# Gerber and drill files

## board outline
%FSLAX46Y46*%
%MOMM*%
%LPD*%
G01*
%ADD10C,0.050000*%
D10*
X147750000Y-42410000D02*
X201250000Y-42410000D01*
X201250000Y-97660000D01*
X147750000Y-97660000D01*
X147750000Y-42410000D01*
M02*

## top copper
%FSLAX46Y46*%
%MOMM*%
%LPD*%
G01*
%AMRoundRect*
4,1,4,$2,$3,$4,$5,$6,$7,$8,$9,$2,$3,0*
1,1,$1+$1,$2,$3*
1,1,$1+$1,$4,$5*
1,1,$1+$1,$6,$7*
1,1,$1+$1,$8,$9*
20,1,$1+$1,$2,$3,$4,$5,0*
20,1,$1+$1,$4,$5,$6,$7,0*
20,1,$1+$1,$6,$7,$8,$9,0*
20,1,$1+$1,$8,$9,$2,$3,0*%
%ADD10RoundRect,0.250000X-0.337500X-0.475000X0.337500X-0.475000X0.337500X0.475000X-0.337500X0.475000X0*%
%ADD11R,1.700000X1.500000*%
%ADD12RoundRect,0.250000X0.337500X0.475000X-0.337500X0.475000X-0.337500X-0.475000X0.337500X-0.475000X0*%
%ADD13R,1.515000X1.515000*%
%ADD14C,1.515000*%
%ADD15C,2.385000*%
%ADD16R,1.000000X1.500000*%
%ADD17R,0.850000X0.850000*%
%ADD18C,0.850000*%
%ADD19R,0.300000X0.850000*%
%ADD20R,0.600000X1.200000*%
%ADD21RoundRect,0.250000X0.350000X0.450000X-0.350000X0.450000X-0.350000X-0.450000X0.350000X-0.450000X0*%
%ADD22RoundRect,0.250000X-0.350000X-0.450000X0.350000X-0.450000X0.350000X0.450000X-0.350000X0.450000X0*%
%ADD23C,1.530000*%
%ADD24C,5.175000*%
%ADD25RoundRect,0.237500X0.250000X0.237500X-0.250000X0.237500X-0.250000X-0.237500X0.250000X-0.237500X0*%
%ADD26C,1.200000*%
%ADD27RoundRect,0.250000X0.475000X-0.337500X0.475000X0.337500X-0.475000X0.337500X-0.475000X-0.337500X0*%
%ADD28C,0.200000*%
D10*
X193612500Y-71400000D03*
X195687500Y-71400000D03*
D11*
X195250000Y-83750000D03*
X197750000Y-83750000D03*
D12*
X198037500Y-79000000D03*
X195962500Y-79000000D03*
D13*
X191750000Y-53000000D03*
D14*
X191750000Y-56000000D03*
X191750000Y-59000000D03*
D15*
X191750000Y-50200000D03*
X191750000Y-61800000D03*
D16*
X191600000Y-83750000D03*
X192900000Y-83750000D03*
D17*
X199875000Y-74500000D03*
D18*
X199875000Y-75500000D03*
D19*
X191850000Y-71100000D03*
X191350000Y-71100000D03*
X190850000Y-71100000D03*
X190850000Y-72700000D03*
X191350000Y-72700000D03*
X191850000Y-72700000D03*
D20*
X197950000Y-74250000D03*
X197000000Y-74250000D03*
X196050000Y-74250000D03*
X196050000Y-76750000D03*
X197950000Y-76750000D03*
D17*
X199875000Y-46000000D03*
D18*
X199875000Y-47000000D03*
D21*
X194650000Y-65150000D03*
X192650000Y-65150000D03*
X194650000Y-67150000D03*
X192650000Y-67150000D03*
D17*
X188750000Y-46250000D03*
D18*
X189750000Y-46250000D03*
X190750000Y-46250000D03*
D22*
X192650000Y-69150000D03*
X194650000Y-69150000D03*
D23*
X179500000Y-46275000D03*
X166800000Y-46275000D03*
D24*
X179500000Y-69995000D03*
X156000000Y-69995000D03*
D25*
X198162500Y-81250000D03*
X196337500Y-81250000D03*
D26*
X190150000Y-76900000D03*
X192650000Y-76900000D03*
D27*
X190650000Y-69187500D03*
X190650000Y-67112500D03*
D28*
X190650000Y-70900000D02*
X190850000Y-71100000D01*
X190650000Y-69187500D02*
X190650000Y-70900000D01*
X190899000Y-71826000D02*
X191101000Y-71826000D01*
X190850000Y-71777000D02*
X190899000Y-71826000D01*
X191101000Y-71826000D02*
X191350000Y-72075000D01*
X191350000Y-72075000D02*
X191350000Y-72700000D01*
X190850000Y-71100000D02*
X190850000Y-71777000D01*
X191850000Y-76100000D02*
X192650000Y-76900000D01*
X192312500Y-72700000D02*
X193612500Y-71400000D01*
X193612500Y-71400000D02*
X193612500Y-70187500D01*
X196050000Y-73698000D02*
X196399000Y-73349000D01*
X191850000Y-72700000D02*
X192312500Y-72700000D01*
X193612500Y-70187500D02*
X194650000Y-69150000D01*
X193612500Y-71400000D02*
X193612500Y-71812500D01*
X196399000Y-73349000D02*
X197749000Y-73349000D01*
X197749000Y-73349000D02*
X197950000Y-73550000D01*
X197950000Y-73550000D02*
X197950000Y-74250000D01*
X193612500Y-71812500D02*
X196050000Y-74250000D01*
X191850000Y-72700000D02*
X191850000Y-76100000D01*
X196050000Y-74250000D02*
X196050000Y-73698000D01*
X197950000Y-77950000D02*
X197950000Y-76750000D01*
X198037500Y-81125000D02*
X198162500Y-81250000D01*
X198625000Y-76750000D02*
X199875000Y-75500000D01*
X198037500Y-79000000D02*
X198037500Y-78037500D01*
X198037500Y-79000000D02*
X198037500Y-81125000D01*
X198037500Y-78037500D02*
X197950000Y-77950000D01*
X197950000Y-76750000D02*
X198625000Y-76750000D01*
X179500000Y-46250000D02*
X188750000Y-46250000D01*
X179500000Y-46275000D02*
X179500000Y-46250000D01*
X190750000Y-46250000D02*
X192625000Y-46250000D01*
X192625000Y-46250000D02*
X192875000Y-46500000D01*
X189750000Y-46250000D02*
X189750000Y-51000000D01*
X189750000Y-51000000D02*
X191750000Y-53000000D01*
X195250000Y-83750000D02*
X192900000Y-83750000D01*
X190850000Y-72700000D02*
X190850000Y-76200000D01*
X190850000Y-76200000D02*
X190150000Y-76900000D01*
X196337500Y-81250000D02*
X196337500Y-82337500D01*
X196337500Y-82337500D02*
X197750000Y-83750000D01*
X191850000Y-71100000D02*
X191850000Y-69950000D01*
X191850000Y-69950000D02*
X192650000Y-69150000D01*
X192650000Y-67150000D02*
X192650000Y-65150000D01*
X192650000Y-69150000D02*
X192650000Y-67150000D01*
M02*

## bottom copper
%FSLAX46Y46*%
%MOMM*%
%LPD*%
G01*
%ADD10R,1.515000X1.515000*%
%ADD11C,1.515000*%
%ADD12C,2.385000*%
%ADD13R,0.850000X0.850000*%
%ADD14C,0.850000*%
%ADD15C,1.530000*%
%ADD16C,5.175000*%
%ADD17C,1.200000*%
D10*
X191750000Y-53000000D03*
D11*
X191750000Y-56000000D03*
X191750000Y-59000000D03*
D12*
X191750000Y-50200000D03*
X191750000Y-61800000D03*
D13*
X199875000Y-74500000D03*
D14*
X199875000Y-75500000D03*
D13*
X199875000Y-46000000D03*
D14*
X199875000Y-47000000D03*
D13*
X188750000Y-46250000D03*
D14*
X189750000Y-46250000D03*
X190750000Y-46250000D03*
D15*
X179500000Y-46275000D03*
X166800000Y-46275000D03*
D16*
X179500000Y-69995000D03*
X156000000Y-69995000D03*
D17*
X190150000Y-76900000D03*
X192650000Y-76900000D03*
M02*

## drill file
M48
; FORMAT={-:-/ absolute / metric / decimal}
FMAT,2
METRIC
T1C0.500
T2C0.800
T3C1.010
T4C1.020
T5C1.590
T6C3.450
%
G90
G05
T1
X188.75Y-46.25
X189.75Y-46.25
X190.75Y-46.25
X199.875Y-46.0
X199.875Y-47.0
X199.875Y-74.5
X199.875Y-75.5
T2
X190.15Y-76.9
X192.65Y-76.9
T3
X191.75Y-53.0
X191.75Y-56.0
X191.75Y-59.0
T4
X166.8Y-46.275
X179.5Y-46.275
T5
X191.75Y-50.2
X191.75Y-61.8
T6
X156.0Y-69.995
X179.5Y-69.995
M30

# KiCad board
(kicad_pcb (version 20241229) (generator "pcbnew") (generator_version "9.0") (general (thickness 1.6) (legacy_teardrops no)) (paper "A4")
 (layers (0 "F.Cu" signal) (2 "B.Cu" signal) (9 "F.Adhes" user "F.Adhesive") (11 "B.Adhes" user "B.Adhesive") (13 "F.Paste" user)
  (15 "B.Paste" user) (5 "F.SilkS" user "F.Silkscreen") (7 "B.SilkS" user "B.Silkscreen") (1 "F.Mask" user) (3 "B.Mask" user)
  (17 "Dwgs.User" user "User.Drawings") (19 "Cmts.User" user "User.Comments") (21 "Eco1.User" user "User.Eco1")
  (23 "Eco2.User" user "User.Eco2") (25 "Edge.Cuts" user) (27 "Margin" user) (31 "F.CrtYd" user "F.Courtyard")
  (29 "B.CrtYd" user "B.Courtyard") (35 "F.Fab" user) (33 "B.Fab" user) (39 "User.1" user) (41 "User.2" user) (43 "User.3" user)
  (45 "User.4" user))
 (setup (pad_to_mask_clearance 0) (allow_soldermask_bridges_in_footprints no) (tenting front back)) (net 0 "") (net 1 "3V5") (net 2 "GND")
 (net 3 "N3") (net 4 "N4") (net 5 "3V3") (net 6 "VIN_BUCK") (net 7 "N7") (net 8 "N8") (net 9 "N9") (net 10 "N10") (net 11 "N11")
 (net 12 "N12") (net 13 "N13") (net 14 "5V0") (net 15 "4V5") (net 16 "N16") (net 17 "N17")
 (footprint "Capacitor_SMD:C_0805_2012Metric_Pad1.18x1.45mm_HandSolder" (layer "F.Cu") (at 194.65 71.4)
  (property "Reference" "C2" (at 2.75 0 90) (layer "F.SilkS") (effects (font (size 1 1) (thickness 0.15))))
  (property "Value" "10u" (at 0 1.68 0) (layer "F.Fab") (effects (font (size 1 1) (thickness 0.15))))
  (pad "1" smd roundrect (at -1.0375 0) (size 1.175 1.45) (layers "F.Cu" "F.Mask" "F.Paste") (roundrect_rratio 0.212766) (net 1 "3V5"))
  (pad "2" smd roundrect (at 1.0375 0) (size 1.175 1.45) (layers "F.Cu" "F.Mask" "F.Paste") (roundrect_rratio 0.212766) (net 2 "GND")))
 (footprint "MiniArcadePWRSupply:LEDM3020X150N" (layer "F.Cu") (at 196.5 83.75)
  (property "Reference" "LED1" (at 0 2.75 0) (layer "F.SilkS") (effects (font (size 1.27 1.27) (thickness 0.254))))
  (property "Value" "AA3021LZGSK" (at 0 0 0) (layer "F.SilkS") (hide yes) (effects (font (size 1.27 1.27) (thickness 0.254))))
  (pad "1" smd rect (at -1.25 0 90) (size 1.5 1.7) (layers "F.Cu" "F.Mask" "F.Paste") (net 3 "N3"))
  (pad "2" smd rect (at 1.25 0 90) (size 1.5 1.7) (layers "F.Cu" "F.Mask" "F.Paste") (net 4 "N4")))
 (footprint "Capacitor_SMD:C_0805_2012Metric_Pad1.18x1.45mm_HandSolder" (layer "F.Cu") (at 197 79 180)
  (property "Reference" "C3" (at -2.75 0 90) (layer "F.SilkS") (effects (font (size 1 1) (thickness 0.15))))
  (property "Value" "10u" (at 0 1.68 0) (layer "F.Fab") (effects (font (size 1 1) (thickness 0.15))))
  (pad "1" smd roundrect (at -1.0375 0 180) (size 1.175 1.45) (layers "F.Cu" "F.Mask" "F.Paste") (roundrect_rratio 0.212766) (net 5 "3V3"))
  (pad "2" smd roundrect (at 1.0375 0 180) (size 1.175 1.45) (layers "F.Cu" "F.Mask" "F.Paste") (roundrect_rratio 0.212766) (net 2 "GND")))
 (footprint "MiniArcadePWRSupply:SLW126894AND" (layer "F.Cu") (at 191.75 53 -90)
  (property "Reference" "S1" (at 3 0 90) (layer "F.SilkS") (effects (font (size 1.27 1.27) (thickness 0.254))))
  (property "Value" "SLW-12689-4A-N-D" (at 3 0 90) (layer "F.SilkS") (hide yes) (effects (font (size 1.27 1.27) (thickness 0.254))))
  (pad "1" thru_hole rect (at 0 0 270) (size 1.515 1.515) (drill 1.01) (layers "*.Cu" "*.Mask") (remove_unused_layers no) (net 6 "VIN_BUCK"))
  (pad "2" thru_hole circle (at 3 0 270) (size 1.515 1.515) (drill 1.01) (layers "*.Cu" "*.Mask") (remove_unused_layers no) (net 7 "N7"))
  (pad "3" thru_hole circle (at 6 0 270) (size 1.515 1.515) (drill 1.01) (layers "*.Cu" "*.Mask") (remove_unused_layers no) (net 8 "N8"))
  (pad "4" thru_hole circle (at -2.8 0 270) (size 2.385 2.385) (drill 1.59) (layers "*.Cu" "*.Mask") (remove_unused_layers no) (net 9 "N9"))
  (pad "5" thru_hole circle (at 8.8 0 270) (size 2.385 2.385) (drill 1.59) (layers "*.Cu" "*.Mask") (remove_unused_layers no) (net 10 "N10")))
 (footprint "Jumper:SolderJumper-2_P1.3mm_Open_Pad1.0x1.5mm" (layer "F.Cu") (at 192.25 83.75)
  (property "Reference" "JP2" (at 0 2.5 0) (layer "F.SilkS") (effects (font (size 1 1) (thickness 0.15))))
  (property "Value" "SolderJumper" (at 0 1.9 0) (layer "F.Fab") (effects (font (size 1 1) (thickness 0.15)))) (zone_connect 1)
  (pad "1" smd rect (at -0.65 0) (size 1 1.5) (layers "F.Cu" "F.Mask") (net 2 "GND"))
  (pad "2" smd rect (at 0.65 0) (size 1 1.5) (layers "F.Cu" "F.Mask") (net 3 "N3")))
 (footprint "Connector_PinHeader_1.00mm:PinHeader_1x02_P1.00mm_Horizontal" (layer "F.Cu") (at 199.875 74.5)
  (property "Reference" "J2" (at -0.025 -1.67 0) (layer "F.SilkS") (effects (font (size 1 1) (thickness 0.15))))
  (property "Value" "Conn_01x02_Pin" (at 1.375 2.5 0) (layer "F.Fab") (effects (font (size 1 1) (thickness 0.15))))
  (pad "1" thru_hole rect (at 0 0) (size 0.85 0.85) (drill 0.5) (layers "*.Cu" "*.Mask") (remove_unused_layers no) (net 2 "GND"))
  (pad "2" thru_hole circle (at 0 1) (size 0.85 0.85) (drill 0.5) (layers "*.Cu" "*.Mask") (remove_unused_layers no) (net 5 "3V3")))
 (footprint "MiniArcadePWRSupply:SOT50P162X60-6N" (layer "F.Cu") (at 191.35 71.9 -90)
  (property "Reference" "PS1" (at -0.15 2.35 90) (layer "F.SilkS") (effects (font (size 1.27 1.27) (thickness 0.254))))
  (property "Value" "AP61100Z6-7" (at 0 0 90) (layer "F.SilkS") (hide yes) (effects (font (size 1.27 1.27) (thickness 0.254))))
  (pad "1" smd rect (at -0.8 -0.5) (size 0.3 0.85) (layers "F.Cu" "F.Mask" "F.Paste") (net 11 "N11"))
  (pad "2" smd rect (at -0.8 0) (size 0.3 0.85) (layers "F.Cu" "F.Mask" "F.Paste") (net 2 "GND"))
  (pad "3" smd rect (at -0.8 0.5) (size 0.3 0.85) (layers "F.Cu" "F.Mask" "F.Paste") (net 7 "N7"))
  (pad "4" smd rect (at 0.8 0.5) (size 0.3 0.85) (layers "F.Cu" "F.Mask" "F.Paste") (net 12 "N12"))
  (pad "5" smd rect (at 0.8 0) (size 0.3 0.85) (layers "F.Cu" "F.Mask" "F.Paste") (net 7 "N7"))
  (pad "6" smd rect (at 0.8 -0.5) (size 0.3 0.85) (layers "F.Cu" "F.Mask" "F.Paste") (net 1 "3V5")))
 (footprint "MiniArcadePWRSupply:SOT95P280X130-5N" (layer "F.Cu") (at 197 75.5 -90)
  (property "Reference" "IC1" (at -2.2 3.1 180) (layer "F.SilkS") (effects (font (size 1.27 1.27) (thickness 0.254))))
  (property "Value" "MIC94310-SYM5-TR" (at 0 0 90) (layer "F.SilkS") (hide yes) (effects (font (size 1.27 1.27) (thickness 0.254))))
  (pad "1" smd rect (at -1.25 -0.95) (size 0.6 1.2) (layers "F.Cu" "F.Mask" "F.Paste") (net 1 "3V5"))
  (pad "2" smd rect (at -1.25 0) (size 0.6 1.2) (layers "F.Cu" "F.Mask" "F.Paste") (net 2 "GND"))
  (pad "3" smd rect (at -1.25 0.95) (size 0.6 1.2) (layers "F.Cu" "F.Mask" "F.Paste") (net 1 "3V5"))
  (pad "4" smd rect (at 1.25 0.95) (size 0.6 1.2) (layers "F.Cu" "F.Mask" "F.Paste") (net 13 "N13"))
  (pad "5" smd rect (at 1.25 -0.95) (size 0.6 1.2) (layers "F.Cu" "F.Mask" "F.Paste") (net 5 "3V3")))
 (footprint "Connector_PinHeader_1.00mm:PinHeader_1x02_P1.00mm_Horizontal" (layer "F.Cu") (at 199.875 46)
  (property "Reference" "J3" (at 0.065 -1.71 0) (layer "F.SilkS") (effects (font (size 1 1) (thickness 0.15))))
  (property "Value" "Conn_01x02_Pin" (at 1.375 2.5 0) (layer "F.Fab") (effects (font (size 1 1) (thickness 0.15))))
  (pad "1" thru_hole rect (at 0 0) (size 0.85 0.85) (drill 0.5) (layers "*.Cu" "*.Mask") (remove_unused_layers no) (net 2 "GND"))
  (pad "2" thru_hole circle (at 0 1) (size 0.85 0.85) (drill 0.5) (layers "*.Cu" "*.Mask") (remove_unused_layers no) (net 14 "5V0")))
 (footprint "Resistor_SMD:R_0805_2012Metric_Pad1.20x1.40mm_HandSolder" (layer "F.Cu") (at 193.65 65.15 180)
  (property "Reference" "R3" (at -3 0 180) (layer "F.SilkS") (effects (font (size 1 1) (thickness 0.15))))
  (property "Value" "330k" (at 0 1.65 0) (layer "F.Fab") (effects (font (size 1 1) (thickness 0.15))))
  (pad "1" smd roundrect (at -1 0 180) (size 1.2 1.4) (layers "F.Cu" "F.Mask" "F.Paste") (roundrect_rratio 0.208333) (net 2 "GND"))
  (pad "2" smd roundrect (at 1 0 180) (size 1.2 1.4) (layers "F.Cu" "F.Mask" "F.Paste") (roundrect_rratio 0.208333) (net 11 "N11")))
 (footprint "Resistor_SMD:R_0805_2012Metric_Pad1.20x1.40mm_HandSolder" (layer "F.Cu") (at 193.65 67.15 180)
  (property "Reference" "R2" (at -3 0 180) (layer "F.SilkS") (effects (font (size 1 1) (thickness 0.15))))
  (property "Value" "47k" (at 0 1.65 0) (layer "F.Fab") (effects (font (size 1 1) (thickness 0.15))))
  (pad "1" smd roundrect (at -1 0 180) (size 1.2 1.4) (layers "F.Cu" "F.Mask" "F.Paste") (roundrect_rratio 0.208333) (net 2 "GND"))
  (pad "2" smd roundrect (at 1 0 180) (size 1.2 1.4) (layers "F.Cu" "F.Mask" "F.Paste") (roundrect_rratio 0.208333) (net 11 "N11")))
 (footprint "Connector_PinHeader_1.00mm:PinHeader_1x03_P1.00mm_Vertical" (layer "F.Cu") (at 188.75 46.25 90)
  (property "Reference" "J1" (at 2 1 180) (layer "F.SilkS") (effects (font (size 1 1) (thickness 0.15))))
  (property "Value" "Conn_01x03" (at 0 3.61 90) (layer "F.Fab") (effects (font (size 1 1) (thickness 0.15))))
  (pad "1" thru_hole rect (at 0 0 90) (size 0.85 0.85) (drill 0.5) (layers "*.Cu" "*.Mask") (remove_unused_layers no) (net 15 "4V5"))
  (pad "2" thru_hole circle (at 0 1 90) (size 0.85 0.85) (drill 0.5) (layers "*.Cu" "*.Mask") (remove_unused_layers no) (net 6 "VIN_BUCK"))
  (pad "3" thru_hole circle (at 0 2 90) (size 0.85 0.85) (drill 0.5) (layers "*.Cu" "*.Mask") (remove_unused_layers no) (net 14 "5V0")))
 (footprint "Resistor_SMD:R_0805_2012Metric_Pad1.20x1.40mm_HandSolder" (layer "F.Cu") (at 193.65 69.15)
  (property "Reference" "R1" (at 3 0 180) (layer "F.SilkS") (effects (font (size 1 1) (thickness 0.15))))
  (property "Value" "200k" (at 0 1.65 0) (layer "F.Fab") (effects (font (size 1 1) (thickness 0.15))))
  (pad "1" smd roundrect (at -1 0) (size 1.2 1.4) (layers "F.Cu" "F.Mask" "F.Paste") (roundrect_rratio 0.208333) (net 11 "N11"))
  (pad "2" smd roundrect (at 1 0) (size 1.2 1.4) (layers "F.Cu" "F.Mask" "F.Paste") (roundrect_rratio 0.208333) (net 1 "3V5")))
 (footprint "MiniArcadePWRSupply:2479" (layer "F.Cu") (at 167.75 70 90)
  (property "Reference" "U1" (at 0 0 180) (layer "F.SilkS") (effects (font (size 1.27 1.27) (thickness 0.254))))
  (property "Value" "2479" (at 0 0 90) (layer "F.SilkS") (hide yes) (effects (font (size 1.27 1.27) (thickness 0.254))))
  (pad "1" thru_hole circle (at 23.725 11.75 90) (size 1.53 1.53) (drill 1.02) (layers "*.Cu" "*.Mask") (remove_unused_layers no)
   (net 15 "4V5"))
  (pad "2" thru_hole circle (at 23.725 -0.95 90) (size 1.53 1.53) (drill 1.02) (layers "*.Cu" "*.Mask") (remove_unused_layers no)
   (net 2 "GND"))
  (pad "3" thru_hole circle (at 0.005 11.75 90) (size 5.175 5.175) (drill 3.45) (layers "*.Cu" "*.Mask") (remove_unused_layers no)
   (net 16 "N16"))
  (pad "4" thru_hole circle (at 0.005 -11.75 90) (size 5.175 5.175) (drill 3.45) (layers "*.Cu" "*.Mask") (remove_unused_layers no)
   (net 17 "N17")))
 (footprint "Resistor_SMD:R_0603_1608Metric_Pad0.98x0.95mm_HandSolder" (layer "F.Cu") (at 197.25 81.25 180)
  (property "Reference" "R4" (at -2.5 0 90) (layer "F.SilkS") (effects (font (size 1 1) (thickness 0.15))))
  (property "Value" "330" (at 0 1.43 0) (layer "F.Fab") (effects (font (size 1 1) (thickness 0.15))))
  (pad "1" smd roundrect (at -0.9125 0 180) (size 0.975 0.95) (layers "F.Cu" "F.Mask" "F.Paste") (roundrect_rratio 0.25) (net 5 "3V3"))
  (pad "2" smd roundrect (at 0.9125 0 180) (size 0.975 0.95) (layers "F.Cu" "F.Mask" "F.Paste") (roundrect_rratio 0.25) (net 4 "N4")))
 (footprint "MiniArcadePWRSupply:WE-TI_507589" (layer "F.Cu") (at 191.4 76.9)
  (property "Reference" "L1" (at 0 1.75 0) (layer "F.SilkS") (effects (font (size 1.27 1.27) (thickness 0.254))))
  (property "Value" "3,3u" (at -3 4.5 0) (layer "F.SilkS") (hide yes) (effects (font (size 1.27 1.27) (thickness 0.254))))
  (pad "1" thru_hole circle (at -1.25 0) (size 1.2 1.2) (drill 0.8) (layers "*.Cu" "*.Mask") (remove_unused_layers no) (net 12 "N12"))
  (pad "2" thru_hole circle (at 1.25 0) (size 1.2 1.2) (drill 0.8) (layers "*.Cu" "*.Mask") (remove_unused_layers no) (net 1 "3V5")))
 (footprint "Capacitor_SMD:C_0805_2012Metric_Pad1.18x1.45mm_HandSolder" (layer "F.Cu") (at 190.65 68.15 90)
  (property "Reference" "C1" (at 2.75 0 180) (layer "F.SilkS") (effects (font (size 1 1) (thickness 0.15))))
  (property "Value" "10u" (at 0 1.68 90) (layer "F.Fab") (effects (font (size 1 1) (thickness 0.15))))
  (pad "1" smd roundrect (at -1.0375 0 90) (size 1.175 1.45) (layers "F.Cu" "F.Mask" "F.Paste") (roundrect_rratio 0.212766) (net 7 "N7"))
  (pad "2" smd roundrect (at 1.0375 0 90) (size 1.175 1.45) (layers "F.Cu" "F.Mask" "F.Paste") (roundrect_rratio 0.212766) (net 2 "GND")))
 (gr_rect (start 147.75 42.41) (end 201.25 97.66) (stroke (width 0.05) (type default)) (fill no) (layer "Edge.Cuts"))
 (segment (start 190.65 70.9) (end 190.85 71.1) (width 0.2) (layer "F.Cu") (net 7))
 (segment (start 190.65 69.1875) (end 190.65 70.9) (width 0.2) (layer "F.Cu") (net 7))
 (segment (start 190.899 71.826) (end 191.101 71.826) (width 0.2) (layer "F.Cu") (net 7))
 (segment (start 190.85 71.777) (end 190.899 71.826) (width 0.2) (layer "F.Cu") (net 7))
 (segment (start 191.101 71.826) (end 191.35 72.075) (width 0.2) (layer "F.Cu") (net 7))
 (segment (start 191.35 72.075) (end 191.35 72.7) (width 0.2) (layer "F.Cu") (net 7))
 (segment (start 190.85 71.1) (end 190.85 71.777) (width 0.2) (layer "F.Cu") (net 7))
 (segment (start 191.85 76.1) (end 192.65 76.9) (width 0.2) (layer "F.Cu") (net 1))
 (segment (start 192.3125 72.7) (end 193.6125 71.4) (width 0.2) (layer "F.Cu") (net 1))
 (segment (start 193.6125 71.4) (end 193.6125 70.1875) (width 0.2) (layer "F.Cu") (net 1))
 (segment (start 196.05 73.698) (end 196.399 73.349) (width 0.2) (layer "F.Cu") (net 1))
 (segment (start 191.85 72.7) (end 192.3125 72.7) (width 0.2) (layer "F.Cu") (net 1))
 (segment (start 193.6125 70.1875) (end 194.65 69.15) (width 0.2) (layer "F.Cu") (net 1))
 (segment (start 193.6125 71.4) (end 193.6125 71.8125) (width 0.2) (layer "F.Cu") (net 1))
 (segment (start 196.399 73.349) (end 197.749 73.349) (width 0.2) (layer "F.Cu") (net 1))
 (segment (start 197.749 73.349) (end 197.95 73.55) (width 0.2) (layer "F.Cu") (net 1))
 (segment (start 197.95 73.55) (end 197.95 74.25) (width 0.2) (layer "F.Cu") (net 1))
 (segment (start 193.6125 71.8125) (end 196.05 74.25) (width 0.2) (layer "F.Cu") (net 1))
 (segment (start 191.85 72.7) (end 191.85 76.1) (width 0.2) (layer "F.Cu") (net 1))
 (segment (start 196.05 74.25) (end 196.05 73.698) (width 0.2) (layer "F.Cu") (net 1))
 (segment (start 197.95 77.95) (end 197.95 76.75) (width 0.2) (layer "F.Cu") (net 5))
 (segment (start 198.0375 81.125) (end 198.1625 81.25) (width 0.2) (layer "F.Cu") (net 5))
 (segment (start 198.625 76.75) (end 199.875 75.5) (width 0.2) (layer "F.Cu") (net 5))
 (segment (start 198.0375 79) (end 198.0375 78.0375) (width 0.2) (layer "F.Cu") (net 5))
 (segment (start 198.0375 79) (end 198.0375 81.125) (width 0.2) (layer "F.Cu") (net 5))
 (segment (start 198.0375 78.0375) (end 197.95 77.95) (width 0.2) (layer "F.Cu") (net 5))
 (segment (start 197.95 76.75) (end 198.625 76.75) (width 0.2) (layer "F.Cu") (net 5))
 (segment (start 179.5 46.25) (end 188.75 46.25) (width 0.2) (layer "F.Cu") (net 15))
 (segment (start 179.5 46.275) (end 179.5 46.25) (width 0.2) (layer "F.Cu") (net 15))
 (segment (start 190.75 46.25) (end 192.625 46.25) (width 0.2) (layer "F.Cu") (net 14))
 (segment (start 192.625 46.25) (end 192.875 46.5) (width 0.2) (layer "F.Cu") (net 14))
 (segment (start 189.75 46.25) (end 189.75 51) (width 0.2) (layer "F.Cu") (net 6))
 (segment (start 189.75 51) (end 191.75 53) (width 0.2) (layer "F.Cu") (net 6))
 (segment (start 195.25 83.75) (end 192.9 83.75) (width 0.2) (layer "F.Cu") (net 3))
 (segment (start 190.85 72.7) (end 190.85 76.2) (width 0.2) (layer "F.Cu") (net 12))
 (segment (start 190.85 76.2) (end 190.15 76.9) (width 0.2) (layer "F.Cu") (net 12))
 (segment (start 196.3375 81.25) (end 196.3375 82.3375) (width 0.2) (layer "F.Cu") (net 4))
 (segment (start 196.3375 82.3375) (end 197.75 83.75) (width 0.2) (layer "F.Cu") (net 4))
 (segment (start 191.85 71.1) (end 191.85 69.95) (width 0.2) (layer "F.Cu") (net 11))
 (segment (start 191.85 69.95) (end 192.65 69.15) (width 0.2) (layer "F.Cu") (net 11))
 (segment (start 192.65 67.15) (end 192.65 65.15) (width 0.2) (layer "F.Cu") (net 11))
 (segment (start 192.65 69.15) (end 192.65 67.15) (width 0.2) (layer "F.Cu") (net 11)))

